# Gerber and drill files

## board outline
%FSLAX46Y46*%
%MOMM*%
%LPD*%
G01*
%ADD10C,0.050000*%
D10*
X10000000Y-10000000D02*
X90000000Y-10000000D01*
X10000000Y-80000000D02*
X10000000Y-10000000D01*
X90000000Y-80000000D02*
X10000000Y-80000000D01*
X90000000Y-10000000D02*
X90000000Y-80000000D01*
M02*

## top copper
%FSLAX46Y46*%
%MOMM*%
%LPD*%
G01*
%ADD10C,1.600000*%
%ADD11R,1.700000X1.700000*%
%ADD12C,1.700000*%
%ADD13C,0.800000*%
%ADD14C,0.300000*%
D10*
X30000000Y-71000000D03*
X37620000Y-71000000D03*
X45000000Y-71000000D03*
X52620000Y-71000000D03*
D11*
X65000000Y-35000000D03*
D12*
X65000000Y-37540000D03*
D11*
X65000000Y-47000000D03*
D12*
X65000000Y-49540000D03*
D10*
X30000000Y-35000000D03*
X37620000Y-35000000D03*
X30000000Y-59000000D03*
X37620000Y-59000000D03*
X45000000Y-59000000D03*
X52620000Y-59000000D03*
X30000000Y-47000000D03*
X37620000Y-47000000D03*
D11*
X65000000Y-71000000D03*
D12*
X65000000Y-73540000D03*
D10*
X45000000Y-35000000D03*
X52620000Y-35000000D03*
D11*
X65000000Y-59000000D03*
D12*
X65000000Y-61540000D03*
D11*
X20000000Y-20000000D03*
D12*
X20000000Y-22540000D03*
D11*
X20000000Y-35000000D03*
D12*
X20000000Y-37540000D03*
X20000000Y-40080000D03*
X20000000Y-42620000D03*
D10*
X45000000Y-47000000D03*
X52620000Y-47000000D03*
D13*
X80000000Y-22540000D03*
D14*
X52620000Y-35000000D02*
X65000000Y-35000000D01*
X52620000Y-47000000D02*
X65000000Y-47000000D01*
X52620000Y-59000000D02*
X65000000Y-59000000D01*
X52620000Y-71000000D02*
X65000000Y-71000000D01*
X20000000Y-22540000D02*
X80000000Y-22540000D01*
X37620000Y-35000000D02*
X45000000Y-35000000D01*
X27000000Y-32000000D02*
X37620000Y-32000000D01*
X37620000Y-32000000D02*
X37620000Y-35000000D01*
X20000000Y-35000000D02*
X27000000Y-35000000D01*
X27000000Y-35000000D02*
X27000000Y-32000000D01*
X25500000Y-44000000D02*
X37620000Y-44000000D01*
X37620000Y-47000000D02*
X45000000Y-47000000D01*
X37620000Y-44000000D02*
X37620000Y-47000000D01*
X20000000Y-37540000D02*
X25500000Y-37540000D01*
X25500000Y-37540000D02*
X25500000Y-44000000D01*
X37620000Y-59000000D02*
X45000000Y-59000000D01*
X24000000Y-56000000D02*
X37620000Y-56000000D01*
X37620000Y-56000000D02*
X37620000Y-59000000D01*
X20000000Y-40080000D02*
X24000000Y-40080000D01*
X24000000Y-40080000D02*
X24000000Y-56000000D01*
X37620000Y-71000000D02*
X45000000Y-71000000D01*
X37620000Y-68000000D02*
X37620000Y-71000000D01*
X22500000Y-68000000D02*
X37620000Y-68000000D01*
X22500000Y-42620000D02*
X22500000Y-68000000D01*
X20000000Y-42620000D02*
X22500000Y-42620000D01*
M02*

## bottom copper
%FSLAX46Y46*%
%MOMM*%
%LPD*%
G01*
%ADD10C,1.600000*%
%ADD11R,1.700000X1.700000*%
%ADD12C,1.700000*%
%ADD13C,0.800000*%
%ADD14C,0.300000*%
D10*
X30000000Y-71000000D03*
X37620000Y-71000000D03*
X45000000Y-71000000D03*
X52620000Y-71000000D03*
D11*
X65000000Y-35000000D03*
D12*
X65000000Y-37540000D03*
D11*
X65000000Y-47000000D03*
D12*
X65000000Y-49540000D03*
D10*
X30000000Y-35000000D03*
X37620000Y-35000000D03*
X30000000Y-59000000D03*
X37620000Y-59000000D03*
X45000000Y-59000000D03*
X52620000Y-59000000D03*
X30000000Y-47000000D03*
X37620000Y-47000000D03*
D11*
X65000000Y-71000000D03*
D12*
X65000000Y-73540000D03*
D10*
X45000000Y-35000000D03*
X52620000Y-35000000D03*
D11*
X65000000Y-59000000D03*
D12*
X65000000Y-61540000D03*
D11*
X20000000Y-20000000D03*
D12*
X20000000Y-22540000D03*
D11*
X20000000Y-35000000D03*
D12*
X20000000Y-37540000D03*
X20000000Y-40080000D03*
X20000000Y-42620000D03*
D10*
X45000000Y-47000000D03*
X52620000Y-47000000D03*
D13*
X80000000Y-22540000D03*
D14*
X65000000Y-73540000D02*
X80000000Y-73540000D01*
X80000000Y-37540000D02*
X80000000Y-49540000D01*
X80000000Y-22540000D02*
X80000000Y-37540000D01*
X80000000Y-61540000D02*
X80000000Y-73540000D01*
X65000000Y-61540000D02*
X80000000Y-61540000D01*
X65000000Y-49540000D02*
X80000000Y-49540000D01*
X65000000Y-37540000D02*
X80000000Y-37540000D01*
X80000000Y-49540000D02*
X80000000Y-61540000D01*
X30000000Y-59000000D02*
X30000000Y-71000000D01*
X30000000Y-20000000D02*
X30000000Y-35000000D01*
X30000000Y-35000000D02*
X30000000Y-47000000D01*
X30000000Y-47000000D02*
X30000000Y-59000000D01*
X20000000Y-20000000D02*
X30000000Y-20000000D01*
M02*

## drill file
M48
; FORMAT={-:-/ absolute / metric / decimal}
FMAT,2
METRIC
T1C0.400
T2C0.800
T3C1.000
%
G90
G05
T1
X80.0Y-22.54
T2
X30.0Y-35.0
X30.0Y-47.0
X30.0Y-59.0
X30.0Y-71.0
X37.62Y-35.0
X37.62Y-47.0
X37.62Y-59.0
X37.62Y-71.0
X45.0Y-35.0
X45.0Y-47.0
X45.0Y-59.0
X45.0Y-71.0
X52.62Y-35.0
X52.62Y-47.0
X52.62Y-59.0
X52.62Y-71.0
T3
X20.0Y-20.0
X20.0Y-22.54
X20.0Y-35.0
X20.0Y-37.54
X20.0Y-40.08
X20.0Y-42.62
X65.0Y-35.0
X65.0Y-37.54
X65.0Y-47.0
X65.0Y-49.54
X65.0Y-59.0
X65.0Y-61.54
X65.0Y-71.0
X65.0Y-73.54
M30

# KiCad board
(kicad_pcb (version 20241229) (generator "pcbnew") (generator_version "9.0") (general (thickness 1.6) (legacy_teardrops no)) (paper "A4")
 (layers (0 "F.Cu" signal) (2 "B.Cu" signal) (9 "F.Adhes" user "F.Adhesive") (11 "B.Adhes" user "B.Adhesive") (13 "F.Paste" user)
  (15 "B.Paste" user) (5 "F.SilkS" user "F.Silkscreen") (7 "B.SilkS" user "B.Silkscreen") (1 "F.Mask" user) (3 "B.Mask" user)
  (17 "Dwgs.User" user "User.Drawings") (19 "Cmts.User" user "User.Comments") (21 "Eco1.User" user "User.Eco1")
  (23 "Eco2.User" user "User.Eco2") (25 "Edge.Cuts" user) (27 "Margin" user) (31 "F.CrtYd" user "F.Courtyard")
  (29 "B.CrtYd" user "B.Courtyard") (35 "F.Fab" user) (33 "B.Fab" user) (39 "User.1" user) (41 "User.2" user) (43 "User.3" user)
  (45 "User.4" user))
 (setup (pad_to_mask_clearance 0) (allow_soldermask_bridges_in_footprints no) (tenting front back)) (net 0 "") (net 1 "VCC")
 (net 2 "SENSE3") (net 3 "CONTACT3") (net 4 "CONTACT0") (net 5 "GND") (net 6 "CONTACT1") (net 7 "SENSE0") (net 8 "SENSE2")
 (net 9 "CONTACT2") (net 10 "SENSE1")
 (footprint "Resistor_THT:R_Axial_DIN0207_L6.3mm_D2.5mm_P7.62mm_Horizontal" (layer "F.Cu") (at 30 71)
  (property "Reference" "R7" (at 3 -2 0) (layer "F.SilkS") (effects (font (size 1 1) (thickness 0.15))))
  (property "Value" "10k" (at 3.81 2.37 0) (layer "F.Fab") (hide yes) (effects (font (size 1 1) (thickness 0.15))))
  (pad "1" thru_hole circle (at 0 0) (size 1.6 1.6) (drill 0.8) (layers "*.Cu" "*.Mask") (remove_unused_layers no) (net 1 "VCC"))
  (pad "2" thru_hole circle (at 7.62 0) (size 1.6 1.6) (drill 0.8) (layers "*.Cu" "*.Mask") (remove_unused_layers no) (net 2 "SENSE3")))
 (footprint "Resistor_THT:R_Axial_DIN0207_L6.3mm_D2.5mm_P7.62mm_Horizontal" (layer "F.Cu") (at 45 71)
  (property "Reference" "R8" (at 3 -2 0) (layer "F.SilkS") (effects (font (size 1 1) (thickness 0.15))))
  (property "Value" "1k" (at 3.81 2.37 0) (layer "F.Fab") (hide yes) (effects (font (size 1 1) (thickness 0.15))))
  (pad "1" thru_hole circle (at 0 0) (size 1.6 1.6) (drill 0.8) (layers "*.Cu" "*.Mask") (remove_unused_layers no) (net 2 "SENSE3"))
  (pad "2" thru_hole circle (at 7.62 0) (size 1.6 1.6) (drill 0.8) (layers "*.Cu" "*.Mask") (remove_unused_layers no) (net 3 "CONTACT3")))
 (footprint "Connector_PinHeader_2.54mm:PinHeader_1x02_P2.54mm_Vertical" (layer "F.Cu") (at 65 35)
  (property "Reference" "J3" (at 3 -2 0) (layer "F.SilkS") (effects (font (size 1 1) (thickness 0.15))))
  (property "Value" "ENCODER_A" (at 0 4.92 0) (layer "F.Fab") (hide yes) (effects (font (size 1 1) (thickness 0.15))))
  (pad "1" thru_hole rect (at 0 0) (size 1.7 1.7) (drill 1) (layers "*.Cu" "*.Mask") (remove_unused_layers no) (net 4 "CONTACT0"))
  (pad "2" thru_hole circle (at 0 2.54) (size 1.7 1.7) (drill 1) (layers "*.Cu" "*.Mask") (remove_unused_layers no) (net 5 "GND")))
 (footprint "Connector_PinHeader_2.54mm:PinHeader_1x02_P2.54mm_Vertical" (layer "F.Cu") (at 65 47)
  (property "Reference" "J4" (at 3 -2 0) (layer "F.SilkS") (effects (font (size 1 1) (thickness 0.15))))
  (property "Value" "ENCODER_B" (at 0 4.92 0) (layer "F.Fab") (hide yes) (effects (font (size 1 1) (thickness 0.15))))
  (pad "1" thru_hole rect (at 0 0) (size 1.7 1.7) (drill 1) (layers "*.Cu" "*.Mask") (remove_unused_layers no) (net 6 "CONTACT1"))
  (pad "2" thru_hole circle (at 0 2.54) (size 1.7 1.7) (drill 1) (layers "*.Cu" "*.Mask") (remove_unused_layers no) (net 5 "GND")))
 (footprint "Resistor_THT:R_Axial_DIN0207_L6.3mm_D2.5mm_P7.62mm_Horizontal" (layer "F.Cu") (at 30 35)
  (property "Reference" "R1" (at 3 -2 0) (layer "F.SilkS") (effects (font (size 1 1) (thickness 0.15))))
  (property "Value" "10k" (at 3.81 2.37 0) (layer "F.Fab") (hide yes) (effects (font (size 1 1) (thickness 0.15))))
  (pad "1" thru_hole circle (at 0 0) (size 1.6 1.6) (drill 0.8) (layers "*.Cu" "*.Mask") (remove_unused_layers no) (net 1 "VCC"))
  (pad "2" thru_hole circle (at 7.62 0) (size 1.6 1.6) (drill 0.8) (layers "*.Cu" "*.Mask") (remove_unused_layers no) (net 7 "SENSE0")))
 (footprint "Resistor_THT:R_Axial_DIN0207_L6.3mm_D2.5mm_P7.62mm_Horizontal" (layer "F.Cu") (at 30 59)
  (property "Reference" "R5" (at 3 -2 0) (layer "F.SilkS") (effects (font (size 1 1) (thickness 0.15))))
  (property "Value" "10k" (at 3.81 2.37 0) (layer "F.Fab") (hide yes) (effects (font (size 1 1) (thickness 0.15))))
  (pad "1" thru_hole circle (at 0 0) (size 1.6 1.6) (drill 0.8) (layers "*.Cu" "*.Mask") (remove_unused_layers no) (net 1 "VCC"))
  (pad "2" thru_hole circle (at 7.62 0) (size 1.6 1.6) (drill 0.8) (layers "*.Cu" "*.Mask") (remove_unused_layers no) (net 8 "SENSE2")))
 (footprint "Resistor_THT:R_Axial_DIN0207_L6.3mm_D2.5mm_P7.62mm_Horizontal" (layer "F.Cu") (at 45 59)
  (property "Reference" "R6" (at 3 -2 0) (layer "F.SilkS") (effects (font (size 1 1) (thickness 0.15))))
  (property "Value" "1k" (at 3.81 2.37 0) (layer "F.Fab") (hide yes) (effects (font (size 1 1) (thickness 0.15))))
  (pad "1" thru_hole circle (at 0 0) (size 1.6 1.6) (drill 0.8) (layers "*.Cu" "*.Mask") (remove_unused_layers no) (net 8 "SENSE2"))
  (pad "2" thru_hole circle (at 7.62 0) (size 1.6 1.6) (drill 0.8) (layers "*.Cu" "*.Mask") (remove_unused_layers no) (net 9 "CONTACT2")))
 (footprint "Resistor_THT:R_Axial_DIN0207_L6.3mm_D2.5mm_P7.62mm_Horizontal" (layer "F.Cu") (at 30 47)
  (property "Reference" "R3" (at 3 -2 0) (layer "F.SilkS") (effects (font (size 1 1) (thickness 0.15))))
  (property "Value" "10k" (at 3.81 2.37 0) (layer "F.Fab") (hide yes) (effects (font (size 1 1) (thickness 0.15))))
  (pad "1" thru_hole circle (at 0 0) (size 1.6 1.6) (drill 0.8) (layers "*.Cu" "*.Mask") (remove_unused_layers no) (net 1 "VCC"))
  (pad "2" thru_hole circle (at 7.62 0) (size 1.6 1.6) (drill 0.8) (layers "*.Cu" "*.Mask") (remove_unused_layers no) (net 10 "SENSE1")))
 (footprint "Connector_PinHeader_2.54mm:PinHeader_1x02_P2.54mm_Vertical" (layer "F.Cu") (at 65 71)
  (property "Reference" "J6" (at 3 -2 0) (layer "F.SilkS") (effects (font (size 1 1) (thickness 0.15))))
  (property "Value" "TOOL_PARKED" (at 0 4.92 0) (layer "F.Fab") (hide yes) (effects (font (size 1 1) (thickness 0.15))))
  (pad "1" thru_hole rect (at 0 0) (size 1.7 1.7) (drill 1) (layers "*.Cu" "*.Mask") (remove_unused_layers no) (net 3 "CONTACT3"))
  (pad "2" thru_hole circle (at 0 2.54) (size 1.7 1.7) (drill 1) (layers "*.Cu" "*.Mask") (remove_unused_layers no) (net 5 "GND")))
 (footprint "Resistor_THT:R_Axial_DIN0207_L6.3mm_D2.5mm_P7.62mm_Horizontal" (layer "F.Cu") (at 45 35)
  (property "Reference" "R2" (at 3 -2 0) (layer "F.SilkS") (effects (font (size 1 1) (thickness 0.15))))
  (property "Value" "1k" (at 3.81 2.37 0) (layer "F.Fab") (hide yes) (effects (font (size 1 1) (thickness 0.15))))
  (pad "1" thru_hole circle (at 0 0) (size 1.6 1.6) (drill 0.8) (layers "*.Cu" "*.Mask") (remove_unused_layers no) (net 7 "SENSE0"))
  (pad "2" thru_hole circle (at 7.62 0) (size 1.6 1.6) (drill 0.8) (layers "*.Cu" "*.Mask") (remove_unused_layers no) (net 4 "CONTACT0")))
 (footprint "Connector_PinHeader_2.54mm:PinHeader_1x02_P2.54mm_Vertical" (layer "F.Cu") (at 65 59)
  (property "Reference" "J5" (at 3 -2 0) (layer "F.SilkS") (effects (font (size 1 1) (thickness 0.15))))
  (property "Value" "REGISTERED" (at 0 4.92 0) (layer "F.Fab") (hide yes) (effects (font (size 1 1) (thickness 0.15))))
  (pad "1" thru_hole rect (at 0 0) (size 1.7 1.7) (drill 1) (layers "*.Cu" "*.Mask") (remove_unused_layers no) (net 9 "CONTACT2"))
  (pad "2" thru_hole circle (at 0 2.54) (size 1.7 1.7) (drill 1) (layers "*.Cu" "*.Mask") (remove_unused_layers no) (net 5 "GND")))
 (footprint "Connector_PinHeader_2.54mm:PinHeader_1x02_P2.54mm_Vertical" (layer "F.Cu") (at 20 20)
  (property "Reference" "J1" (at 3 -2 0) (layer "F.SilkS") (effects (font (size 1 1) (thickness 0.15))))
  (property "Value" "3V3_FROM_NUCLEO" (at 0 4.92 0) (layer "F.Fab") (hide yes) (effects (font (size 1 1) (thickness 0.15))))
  (pad "1" thru_hole rect (at 0 0) (size 1.7 1.7) (drill 1) (layers "*.Cu" "*.Mask") (remove_unused_layers no) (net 1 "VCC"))
  (pad "2" thru_hole circle (at 0 2.54) (size 1.7 1.7) (drill 1) (layers "*.Cu" "*.Mask") (remove_unused_layers no) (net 5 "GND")))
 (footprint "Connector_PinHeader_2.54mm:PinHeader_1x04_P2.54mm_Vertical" (layer "F.Cu") (at 20 35)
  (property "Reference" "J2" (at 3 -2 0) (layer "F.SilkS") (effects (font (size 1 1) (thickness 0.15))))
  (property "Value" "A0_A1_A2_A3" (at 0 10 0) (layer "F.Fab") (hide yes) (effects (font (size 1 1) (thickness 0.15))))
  (pad "1" thru_hole rect (at 0 0) (size 1.7 1.7) (drill 1) (layers "*.Cu" "*.Mask") (remove_unused_layers no) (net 7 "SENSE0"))
  (pad "2" thru_hole circle (at 0 2.54) (size 1.7 1.7) (drill 1) (layers "*.Cu" "*.Mask") (remove_unused_layers no) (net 10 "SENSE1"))
  (pad "3" thru_hole circle (at 0 5.08) (size 1.7 1.7) (drill 1) (layers "*.Cu" "*.Mask") (remove_unused_layers no) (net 8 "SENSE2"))
  (pad "4" thru_hole circle (at 0 7.62) (size 1.7 1.7) (drill 1) (layers "*.Cu" "*.Mask") (remove_unused_layers no) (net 2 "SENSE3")))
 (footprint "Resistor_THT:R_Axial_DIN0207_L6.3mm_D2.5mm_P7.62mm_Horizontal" (layer "F.Cu") (at 45 47)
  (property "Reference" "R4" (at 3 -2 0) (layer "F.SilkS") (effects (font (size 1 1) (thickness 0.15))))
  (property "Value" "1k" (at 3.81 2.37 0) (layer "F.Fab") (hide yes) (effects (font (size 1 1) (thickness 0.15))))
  (pad "1" thru_hole circle (at 0 0) (size 1.6 1.6) (drill 0.8) (layers "*.Cu" "*.Mask") (remove_unused_layers no) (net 10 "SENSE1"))
  (pad "2" thru_hole circle (at 7.62 0) (size 1.6 1.6) (drill 0.8) (layers "*.Cu" "*.Mask") (remove_unused_layers no) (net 6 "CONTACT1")))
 (gr_line (start 10 10) (end 90 10) (stroke (width 0.05) (type default)) (layer "Edge.Cuts"))
 (gr_line (start 10 80) (end 10 10) (stroke (width 0.05) (type default)) (layer "Edge.Cuts"))
 (gr_line (start 90 80) (end 10 80) (stroke (width 0.05) (type default)) (layer "Edge.Cuts"))
 (gr_line (start 90 10) (end 90 80) (stroke (width 0.05) (type default)) (layer "Edge.Cuts"))
 (segment (start 52.62 35) (end 65 35) (width 0.3) (layer "F.Cu") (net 4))
 (segment (start 52.62 47) (end 65 47) (width 0.3) (layer "F.Cu") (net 6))
 (segment (start 52.62 59) (end 65 59) (width 0.3) (layer "F.Cu") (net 9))
 (segment (start 52.62 71) (end 65 71) (width 0.3) (layer "F.Cu") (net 3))
 (segment (start 20 22.54) (end 80 22.54) (width 0.3) (layer "F.Cu") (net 5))
 (via (at 80 22.54) (size 0.8) (drill 0.4) (layers "F.Cu" "B.Cu") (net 5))
 (segment (start 65 73.54) (end 80 73.54) (width 0.3) (layer "B.Cu") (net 5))
 (segment (start 80 37.54) (end 80 49.54) (width 0.3) (layer "B.Cu") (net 5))
 (segment (start 80 22.54) (end 80 37.54) (width 0.3) (layer "B.Cu") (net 5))
 (segment (start 80 61.54) (end 80 73.54) (width 0.3) (layer "B.Cu") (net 5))
 (segment (start 65 61.54) (end 80 61.54) (width 0.3) (layer "B.Cu") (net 5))
 (segment (start 65 49.54) (end 80 49.54) (width 0.3) (layer "B.Cu") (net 5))
 (segment (start 65 37.54) (end 80 37.54) (width 0.3) (layer "B.Cu") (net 5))
 (segment (start 80 49.54) (end 80 61.54) (width 0.3) (layer "B.Cu") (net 5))
 (segment (start 37.62 35) (end 45 35) (width 0.3) (layer "F.Cu") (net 7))
 (segment (start 27 32) (end 37.62 32) (width 0.3) (layer "F.Cu") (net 7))
 (segment (start 37.62 32) (end 37.62 35) (width 0.3) (layer "F.Cu") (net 7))
 (segment (start 20 35) (end 27 35) (width 0.3) (layer "F.Cu") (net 7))
 (segment (start 27 35) (end 27 32) (width 0.3) (layer "F.Cu") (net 7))
 (segment (start 25.5 44) (end 37.62 44) (width 0.3) (layer "F.Cu") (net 10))
 (segment (start 37.62 47) (end 45 47) (width 0.3) (layer "F.Cu") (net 10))
 (segment (start 37.62 44) (end 37.62 47) (width 0.3) (layer "F.Cu") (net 10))
 (segment (start 20 37.54) (end 25.5 37.54) (width 0.3) (layer "F.Cu") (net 10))
 (segment (start 25.5 37.54) (end 25.5 44) (width 0.3) (layer "F.Cu") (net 10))
 (segment (start 37.62 59) (end 45 59) (width 0.3) (layer "F.Cu") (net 8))
 (segment (start 24 56) (end 37.62 56) (width 0.3) (layer "F.Cu") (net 8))
 (segment (start 37.62 56) (end 37.62 59) (width 0.3) (layer "F.Cu") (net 8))
 (segment (start 20 40.08) (end 24 40.08) (width 0.3) (layer "F.Cu") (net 8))
 (segment (start 24 40.08) (end 24 56) (width 0.3) (layer "F.Cu") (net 8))
 (segment (start 37.62 71) (end 45 71) (width 0.3) (layer "F.Cu") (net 2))
 (segment (start 37.62 68) (end 37.62 71) (width 0.3) (layer "F.Cu") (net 2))
 (segment (start 22.5 68) (end 37.62 68) (width 0.3) (layer "F.Cu") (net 2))
 (segment (start 22.5 42.62) (end 22.5 68) (width 0.3) (layer "F.Cu") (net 2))
 (segment (start 20 42.62) (end 22.5 42.62) (width 0.3) (layer "F.Cu") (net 2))
 (segment (start 30 59) (end 30 71) (width 0.3) (layer "B.Cu") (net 1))
 (segment (start 30 20) (end 30 35) (width 0.3) (layer "B.Cu") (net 1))
 (segment (start 30 35) (end 30 47) (width 0.3) (layer "B.Cu") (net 1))
 (segment (start 30 47) (end 30 59) (width 0.3) (layer "B.Cu") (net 1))
 (segment (start 20 20) (end 30 20) (width 0.3) (layer "B.Cu") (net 1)))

